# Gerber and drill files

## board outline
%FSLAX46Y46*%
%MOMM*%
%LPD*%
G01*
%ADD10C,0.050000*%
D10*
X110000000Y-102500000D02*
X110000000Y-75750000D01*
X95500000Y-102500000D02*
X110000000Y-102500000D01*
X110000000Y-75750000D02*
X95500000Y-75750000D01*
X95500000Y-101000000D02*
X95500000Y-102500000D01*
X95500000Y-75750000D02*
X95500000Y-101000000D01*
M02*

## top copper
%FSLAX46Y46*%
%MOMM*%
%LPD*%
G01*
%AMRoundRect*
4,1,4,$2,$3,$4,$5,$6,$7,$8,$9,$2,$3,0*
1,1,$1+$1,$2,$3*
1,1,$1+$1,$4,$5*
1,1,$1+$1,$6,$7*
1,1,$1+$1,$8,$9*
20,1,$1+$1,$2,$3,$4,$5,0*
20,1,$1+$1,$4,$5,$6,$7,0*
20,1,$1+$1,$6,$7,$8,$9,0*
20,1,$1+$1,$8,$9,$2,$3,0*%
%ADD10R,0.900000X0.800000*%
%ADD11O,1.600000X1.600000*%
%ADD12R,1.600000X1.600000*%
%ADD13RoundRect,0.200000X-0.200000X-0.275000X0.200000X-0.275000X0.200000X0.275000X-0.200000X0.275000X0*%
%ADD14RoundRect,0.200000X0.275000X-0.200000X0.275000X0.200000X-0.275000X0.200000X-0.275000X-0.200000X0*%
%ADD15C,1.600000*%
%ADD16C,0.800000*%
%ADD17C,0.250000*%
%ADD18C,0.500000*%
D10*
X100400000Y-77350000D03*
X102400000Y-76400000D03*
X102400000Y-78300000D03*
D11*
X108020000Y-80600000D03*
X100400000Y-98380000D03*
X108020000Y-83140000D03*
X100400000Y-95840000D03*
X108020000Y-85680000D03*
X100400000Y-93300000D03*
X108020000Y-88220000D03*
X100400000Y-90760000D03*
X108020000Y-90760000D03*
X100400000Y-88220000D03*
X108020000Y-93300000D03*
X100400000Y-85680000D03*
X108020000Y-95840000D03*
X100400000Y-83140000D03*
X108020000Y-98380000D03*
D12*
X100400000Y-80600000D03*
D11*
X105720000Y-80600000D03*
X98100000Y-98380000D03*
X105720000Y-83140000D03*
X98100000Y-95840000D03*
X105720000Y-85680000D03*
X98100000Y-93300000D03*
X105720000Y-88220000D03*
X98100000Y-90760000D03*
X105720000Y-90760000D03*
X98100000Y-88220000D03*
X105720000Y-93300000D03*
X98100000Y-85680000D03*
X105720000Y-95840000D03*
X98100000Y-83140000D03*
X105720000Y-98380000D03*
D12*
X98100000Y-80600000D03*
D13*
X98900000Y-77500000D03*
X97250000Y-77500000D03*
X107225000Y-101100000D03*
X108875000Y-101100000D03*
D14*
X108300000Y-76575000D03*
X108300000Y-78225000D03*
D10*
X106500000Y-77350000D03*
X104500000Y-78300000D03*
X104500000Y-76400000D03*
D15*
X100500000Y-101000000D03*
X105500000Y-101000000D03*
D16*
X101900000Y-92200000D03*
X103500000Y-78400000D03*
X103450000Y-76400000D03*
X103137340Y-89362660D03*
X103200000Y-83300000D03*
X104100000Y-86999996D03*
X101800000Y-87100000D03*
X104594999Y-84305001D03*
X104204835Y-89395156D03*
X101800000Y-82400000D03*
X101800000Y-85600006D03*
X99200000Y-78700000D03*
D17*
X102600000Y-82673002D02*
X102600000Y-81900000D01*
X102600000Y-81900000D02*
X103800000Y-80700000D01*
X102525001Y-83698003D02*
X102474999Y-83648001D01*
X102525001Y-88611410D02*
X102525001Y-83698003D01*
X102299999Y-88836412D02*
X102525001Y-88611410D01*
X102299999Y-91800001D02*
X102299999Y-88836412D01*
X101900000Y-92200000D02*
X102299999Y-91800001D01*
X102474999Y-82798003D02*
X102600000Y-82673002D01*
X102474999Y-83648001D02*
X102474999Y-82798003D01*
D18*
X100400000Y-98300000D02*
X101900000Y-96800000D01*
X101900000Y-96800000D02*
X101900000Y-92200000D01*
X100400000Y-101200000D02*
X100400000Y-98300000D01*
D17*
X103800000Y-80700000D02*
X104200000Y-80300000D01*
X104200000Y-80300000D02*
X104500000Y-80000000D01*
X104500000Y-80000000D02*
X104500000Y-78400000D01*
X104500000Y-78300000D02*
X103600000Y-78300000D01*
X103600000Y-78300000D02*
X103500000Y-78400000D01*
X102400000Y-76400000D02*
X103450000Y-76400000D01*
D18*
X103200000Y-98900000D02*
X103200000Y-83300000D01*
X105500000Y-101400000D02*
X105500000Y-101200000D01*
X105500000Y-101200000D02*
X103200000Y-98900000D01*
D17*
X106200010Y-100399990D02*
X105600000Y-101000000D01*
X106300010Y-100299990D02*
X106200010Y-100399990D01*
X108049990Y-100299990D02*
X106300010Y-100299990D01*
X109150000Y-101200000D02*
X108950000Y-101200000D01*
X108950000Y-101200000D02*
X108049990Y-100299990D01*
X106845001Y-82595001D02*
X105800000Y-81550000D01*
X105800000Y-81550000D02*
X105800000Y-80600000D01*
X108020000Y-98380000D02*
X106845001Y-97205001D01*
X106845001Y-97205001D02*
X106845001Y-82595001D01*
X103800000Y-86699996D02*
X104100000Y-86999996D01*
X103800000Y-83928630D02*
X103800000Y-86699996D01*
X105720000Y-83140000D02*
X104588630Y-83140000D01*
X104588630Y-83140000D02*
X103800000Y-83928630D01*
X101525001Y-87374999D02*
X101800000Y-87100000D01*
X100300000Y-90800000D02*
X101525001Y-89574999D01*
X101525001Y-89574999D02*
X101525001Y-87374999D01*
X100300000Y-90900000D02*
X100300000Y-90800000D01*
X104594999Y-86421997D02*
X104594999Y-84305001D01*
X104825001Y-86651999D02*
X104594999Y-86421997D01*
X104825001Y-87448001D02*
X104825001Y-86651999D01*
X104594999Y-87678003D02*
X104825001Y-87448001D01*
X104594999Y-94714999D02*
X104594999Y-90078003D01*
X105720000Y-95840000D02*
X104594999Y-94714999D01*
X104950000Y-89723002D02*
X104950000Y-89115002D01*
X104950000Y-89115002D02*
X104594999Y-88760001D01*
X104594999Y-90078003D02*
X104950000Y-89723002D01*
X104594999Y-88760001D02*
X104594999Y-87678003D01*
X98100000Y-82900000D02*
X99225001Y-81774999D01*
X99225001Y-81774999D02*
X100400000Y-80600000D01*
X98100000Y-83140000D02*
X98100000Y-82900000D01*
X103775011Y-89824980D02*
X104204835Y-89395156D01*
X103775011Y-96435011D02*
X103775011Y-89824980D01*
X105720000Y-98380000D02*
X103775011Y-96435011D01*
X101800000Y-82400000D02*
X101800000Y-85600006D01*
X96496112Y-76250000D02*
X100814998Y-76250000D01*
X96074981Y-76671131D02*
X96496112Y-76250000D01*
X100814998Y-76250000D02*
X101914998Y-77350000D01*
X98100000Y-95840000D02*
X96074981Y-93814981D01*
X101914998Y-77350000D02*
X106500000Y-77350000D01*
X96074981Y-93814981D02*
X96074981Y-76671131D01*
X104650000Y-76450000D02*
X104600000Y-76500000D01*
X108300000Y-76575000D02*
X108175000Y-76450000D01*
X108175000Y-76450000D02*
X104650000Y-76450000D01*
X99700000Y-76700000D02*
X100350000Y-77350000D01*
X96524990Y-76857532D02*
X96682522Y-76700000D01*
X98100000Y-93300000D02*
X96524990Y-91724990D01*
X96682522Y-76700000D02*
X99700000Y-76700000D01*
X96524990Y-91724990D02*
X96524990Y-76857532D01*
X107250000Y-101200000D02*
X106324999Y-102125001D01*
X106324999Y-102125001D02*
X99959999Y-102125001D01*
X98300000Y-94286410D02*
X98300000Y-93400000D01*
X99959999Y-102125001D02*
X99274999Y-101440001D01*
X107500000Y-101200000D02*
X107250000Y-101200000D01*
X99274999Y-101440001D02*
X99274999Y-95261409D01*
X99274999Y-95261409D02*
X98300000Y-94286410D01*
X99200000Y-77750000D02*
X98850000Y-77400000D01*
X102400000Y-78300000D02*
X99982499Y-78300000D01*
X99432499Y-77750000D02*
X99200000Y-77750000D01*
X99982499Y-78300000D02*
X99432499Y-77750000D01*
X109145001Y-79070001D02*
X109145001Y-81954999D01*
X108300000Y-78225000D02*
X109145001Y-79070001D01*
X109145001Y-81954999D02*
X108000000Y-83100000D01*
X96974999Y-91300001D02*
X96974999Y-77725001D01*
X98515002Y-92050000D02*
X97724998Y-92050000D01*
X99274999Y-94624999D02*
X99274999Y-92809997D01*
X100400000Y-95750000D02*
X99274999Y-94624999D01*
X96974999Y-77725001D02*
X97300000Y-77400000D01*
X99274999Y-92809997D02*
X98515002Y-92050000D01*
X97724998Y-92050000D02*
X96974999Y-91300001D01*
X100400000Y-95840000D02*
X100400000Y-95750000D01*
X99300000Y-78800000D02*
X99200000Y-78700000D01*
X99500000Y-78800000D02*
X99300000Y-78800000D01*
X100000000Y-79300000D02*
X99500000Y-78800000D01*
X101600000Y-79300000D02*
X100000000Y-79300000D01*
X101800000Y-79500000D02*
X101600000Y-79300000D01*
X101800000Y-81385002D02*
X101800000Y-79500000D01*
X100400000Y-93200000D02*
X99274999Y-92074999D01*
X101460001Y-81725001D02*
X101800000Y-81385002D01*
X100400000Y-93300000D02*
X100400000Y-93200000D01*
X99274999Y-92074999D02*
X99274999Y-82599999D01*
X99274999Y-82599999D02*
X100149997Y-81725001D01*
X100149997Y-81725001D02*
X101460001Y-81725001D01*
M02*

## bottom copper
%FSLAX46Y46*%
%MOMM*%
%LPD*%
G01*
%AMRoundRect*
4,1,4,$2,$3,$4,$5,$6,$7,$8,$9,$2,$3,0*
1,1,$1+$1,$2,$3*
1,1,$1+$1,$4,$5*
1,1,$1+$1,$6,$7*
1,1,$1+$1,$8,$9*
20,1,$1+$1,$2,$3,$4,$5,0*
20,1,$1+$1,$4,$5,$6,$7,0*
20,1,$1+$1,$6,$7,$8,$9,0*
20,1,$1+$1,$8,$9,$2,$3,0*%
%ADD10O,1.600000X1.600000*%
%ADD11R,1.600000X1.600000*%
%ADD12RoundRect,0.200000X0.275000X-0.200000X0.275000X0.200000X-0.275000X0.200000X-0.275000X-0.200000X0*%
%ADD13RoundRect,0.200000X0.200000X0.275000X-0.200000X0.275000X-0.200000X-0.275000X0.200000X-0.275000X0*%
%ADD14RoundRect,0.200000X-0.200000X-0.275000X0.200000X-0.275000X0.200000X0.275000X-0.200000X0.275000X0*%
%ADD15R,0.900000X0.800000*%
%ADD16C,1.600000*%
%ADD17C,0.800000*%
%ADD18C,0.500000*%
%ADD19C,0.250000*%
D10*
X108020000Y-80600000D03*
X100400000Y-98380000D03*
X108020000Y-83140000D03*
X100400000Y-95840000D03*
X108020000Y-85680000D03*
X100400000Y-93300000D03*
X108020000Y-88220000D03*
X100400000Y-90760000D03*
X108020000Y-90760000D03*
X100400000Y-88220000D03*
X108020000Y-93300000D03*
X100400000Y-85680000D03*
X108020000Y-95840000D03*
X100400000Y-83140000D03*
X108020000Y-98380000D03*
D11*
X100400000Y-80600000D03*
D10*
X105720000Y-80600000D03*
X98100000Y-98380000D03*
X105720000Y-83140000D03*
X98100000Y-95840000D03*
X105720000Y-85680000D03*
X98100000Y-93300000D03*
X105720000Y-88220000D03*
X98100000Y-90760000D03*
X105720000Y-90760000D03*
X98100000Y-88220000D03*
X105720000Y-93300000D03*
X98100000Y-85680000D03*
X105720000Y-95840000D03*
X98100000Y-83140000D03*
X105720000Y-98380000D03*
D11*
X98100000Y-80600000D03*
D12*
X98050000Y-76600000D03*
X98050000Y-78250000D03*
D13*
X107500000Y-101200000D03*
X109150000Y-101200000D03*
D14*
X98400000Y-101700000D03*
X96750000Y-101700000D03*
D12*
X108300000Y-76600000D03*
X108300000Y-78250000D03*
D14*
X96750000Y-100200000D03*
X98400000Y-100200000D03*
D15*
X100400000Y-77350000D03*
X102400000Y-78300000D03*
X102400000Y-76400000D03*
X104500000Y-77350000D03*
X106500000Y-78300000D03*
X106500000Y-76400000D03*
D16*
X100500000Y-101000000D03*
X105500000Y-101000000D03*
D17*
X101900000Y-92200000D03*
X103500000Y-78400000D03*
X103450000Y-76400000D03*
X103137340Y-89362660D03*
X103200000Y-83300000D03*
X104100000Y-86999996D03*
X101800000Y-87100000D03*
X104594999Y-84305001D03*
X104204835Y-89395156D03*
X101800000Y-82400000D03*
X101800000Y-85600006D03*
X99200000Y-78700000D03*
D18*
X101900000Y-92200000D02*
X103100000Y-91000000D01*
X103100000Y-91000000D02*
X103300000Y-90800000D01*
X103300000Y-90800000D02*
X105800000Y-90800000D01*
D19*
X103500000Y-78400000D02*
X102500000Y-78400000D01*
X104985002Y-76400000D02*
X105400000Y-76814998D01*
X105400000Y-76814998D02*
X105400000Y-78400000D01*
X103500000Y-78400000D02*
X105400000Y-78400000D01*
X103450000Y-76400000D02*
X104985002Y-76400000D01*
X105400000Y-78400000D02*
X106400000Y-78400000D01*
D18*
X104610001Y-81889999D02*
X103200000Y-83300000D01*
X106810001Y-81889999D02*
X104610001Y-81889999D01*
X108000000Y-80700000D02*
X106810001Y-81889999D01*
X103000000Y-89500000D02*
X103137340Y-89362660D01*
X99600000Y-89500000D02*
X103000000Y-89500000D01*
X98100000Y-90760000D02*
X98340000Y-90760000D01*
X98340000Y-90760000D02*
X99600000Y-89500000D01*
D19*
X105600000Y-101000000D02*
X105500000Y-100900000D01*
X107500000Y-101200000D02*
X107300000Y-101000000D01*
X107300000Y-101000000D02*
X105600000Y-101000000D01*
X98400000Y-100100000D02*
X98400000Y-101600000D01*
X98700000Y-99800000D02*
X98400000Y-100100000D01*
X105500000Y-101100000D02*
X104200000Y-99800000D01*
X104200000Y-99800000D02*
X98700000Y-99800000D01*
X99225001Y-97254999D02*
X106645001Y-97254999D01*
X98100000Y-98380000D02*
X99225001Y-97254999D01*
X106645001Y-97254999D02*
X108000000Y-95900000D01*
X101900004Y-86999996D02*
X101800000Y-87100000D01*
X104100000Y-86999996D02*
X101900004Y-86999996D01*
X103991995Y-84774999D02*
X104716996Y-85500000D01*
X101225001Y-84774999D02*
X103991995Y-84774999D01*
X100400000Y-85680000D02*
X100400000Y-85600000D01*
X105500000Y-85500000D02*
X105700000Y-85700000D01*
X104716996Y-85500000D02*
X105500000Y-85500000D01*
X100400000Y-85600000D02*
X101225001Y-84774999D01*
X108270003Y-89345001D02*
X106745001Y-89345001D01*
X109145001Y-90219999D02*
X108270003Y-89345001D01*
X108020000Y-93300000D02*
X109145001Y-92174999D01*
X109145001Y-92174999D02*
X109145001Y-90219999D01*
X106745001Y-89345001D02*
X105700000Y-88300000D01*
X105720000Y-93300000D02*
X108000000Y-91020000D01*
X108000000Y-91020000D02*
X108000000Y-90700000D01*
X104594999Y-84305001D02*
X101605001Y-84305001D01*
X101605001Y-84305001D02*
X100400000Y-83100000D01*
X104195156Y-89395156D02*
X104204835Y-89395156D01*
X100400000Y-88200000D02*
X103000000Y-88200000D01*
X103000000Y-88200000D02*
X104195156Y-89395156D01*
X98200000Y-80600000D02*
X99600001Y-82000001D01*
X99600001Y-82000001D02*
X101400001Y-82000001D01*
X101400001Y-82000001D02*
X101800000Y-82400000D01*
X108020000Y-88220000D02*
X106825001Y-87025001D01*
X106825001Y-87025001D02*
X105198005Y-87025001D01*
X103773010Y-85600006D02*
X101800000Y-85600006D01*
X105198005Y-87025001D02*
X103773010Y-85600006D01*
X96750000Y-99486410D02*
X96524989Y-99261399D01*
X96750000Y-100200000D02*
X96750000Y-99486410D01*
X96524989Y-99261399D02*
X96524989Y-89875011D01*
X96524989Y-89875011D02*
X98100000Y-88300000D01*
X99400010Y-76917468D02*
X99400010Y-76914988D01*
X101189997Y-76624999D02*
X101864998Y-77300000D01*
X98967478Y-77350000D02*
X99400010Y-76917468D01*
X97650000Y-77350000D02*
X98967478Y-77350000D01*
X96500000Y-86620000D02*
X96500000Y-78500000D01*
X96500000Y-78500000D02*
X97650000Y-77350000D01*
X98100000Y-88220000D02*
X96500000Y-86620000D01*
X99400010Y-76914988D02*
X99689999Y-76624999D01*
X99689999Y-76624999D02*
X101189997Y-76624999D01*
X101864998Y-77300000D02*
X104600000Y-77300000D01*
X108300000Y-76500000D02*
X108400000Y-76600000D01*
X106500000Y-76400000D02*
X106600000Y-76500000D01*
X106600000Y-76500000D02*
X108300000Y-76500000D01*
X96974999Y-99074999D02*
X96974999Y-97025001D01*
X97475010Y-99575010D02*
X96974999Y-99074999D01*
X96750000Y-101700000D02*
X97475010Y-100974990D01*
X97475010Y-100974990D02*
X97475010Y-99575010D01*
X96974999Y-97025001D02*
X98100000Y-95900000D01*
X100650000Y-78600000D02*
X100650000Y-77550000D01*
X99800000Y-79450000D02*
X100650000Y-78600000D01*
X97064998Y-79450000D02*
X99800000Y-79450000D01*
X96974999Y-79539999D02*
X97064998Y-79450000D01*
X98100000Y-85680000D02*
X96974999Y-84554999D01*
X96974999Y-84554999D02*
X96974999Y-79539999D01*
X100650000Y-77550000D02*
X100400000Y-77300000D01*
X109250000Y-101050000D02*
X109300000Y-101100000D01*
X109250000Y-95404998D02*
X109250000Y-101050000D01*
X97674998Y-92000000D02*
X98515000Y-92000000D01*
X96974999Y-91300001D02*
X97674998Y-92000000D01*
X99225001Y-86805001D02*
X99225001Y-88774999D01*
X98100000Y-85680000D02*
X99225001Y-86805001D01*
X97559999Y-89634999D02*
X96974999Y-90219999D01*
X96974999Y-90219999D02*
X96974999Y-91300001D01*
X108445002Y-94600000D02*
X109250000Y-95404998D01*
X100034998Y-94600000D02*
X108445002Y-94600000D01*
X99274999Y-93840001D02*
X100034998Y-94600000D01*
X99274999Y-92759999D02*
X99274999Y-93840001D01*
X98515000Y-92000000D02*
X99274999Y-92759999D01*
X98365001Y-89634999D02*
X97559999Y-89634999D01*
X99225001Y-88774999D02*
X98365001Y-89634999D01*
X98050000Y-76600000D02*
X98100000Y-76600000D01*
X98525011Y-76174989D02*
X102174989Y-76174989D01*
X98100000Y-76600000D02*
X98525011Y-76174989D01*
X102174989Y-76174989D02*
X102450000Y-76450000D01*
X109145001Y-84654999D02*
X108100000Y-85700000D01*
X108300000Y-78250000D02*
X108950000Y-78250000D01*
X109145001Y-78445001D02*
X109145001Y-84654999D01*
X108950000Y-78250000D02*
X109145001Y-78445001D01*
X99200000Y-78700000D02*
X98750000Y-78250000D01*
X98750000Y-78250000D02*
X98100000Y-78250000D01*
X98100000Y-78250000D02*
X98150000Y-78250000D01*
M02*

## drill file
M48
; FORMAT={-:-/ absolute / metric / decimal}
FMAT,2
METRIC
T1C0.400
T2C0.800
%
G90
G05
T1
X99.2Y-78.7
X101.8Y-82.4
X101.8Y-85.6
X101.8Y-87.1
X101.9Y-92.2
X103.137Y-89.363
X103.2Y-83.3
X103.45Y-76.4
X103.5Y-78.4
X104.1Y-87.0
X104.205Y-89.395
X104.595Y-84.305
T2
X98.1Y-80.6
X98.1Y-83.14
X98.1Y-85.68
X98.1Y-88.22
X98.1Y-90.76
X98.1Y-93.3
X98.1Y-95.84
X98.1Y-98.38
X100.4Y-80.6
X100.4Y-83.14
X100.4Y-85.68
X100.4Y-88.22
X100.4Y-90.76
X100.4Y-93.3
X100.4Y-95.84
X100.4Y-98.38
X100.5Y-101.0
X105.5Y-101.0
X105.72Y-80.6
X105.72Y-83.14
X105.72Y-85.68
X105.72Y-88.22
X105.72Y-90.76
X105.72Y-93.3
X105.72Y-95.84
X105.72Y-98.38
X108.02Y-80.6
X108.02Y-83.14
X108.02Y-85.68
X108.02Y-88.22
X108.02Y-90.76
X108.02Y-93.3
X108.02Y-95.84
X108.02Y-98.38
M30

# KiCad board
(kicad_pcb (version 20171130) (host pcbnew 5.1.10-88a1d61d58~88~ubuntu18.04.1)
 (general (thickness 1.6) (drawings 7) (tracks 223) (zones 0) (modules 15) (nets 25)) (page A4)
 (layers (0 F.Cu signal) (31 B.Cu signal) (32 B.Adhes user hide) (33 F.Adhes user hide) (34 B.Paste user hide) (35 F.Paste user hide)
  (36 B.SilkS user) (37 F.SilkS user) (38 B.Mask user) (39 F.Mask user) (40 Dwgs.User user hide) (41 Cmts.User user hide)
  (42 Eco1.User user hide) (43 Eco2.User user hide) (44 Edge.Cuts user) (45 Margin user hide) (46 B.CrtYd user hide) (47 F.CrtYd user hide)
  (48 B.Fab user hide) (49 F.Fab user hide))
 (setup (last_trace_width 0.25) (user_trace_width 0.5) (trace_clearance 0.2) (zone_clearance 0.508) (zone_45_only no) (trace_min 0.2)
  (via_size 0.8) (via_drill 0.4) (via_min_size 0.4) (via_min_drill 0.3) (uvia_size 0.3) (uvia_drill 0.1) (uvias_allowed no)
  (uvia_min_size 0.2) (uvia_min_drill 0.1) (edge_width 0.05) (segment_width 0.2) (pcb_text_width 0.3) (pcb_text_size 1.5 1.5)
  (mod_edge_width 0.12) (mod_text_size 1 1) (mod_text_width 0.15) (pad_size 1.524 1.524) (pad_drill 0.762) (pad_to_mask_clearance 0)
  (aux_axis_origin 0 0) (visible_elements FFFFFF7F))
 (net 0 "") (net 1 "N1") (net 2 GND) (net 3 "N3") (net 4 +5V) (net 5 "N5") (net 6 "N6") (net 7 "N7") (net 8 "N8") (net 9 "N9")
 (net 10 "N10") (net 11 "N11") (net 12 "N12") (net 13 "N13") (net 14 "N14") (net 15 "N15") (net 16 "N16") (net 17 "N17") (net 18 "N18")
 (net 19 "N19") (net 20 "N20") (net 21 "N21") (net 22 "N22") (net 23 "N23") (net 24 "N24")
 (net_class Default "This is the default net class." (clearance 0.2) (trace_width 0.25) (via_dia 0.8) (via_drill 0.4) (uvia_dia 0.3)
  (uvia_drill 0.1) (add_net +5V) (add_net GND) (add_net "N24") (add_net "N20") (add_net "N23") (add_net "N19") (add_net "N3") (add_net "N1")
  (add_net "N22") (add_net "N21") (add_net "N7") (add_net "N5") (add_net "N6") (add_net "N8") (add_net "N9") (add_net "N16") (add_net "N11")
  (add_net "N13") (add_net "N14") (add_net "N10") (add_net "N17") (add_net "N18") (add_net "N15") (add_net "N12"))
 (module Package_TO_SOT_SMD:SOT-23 (layer F.Cu) (at 101.4 77.35 180)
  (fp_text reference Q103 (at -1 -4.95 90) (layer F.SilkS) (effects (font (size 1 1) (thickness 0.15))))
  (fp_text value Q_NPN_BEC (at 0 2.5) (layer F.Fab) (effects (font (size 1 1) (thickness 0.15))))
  (pad 3 smd rect (at 1 0 180) (size 0.9 0.8) (layers F.Cu F.Paste F.Mask) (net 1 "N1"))
  (pad 2 smd rect (at -1 0.95 180) (size 0.9 0.8) (layers F.Cu F.Paste F.Mask) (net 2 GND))
  (pad 1 smd rect (at -1 -0.95 180) (size 0.9 0.8) (layers F.Cu F.Paste F.Mask) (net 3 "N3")))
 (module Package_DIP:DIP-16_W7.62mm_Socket (layer F.Cu) (at 100.4 80.6)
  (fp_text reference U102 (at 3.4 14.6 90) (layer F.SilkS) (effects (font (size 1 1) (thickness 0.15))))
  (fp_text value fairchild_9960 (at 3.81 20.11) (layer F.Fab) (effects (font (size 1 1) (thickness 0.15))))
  (pad 16 thru_hole oval (at 7.62 0) (size 1.6 1.6) (drill 0.8) (layers *.Cu *.Mask) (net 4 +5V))
  (pad 8 thru_hole oval (at 0 17.78) (size 1.6 1.6) (drill 0.8) (layers *.Cu *.Mask) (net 2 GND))
  (pad 15 thru_hole oval (at 7.62 2.54) (size 1.6 1.6) (drill 0.8) (layers *.Cu *.Mask) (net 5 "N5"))
  (pad 7 thru_hole oval (at 0 15.24) (size 1.6 1.6) (drill 0.8) (layers *.Cu *.Mask) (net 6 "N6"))
  (pad 14 thru_hole oval (at 7.62 5.08) (size 1.6 1.6) (drill 0.8) (layers *.Cu *.Mask) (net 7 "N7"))
  (pad 6 thru_hole oval (at 0 12.7) (size 1.6 1.6) (drill 0.8) (layers *.Cu *.Mask) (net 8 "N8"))
  (pad 13 thru_hole oval (at 7.62 7.62) (size 1.6 1.6) (drill 0.8) (layers *.Cu *.Mask) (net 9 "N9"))
  (pad 5 thru_hole oval (at 0 10.16) (size 1.6 1.6) (drill 0.8) (layers *.Cu *.Mask) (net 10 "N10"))
  (pad 12 thru_hole oval (at 7.62 10.16) (size 1.6 1.6) (drill 0.8) (layers *.Cu *.Mask) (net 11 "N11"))
  (pad 4 thru_hole oval (at 0 7.62) (size 1.6 1.6) (drill 0.8) (layers *.Cu *.Mask) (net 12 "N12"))
  (pad 11 thru_hole oval (at 7.62 12.7) (size 1.6 1.6) (drill 0.8) (layers *.Cu *.Mask) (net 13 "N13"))
  (pad 3 thru_hole oval (at 0 5.08) (size 1.6 1.6) (drill 0.8) (layers *.Cu *.Mask) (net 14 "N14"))
  (pad 10 thru_hole oval (at 7.62 15.24) (size 1.6 1.6) (drill 0.8) (layers *.Cu *.Mask) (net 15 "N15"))
  (pad 2 thru_hole oval (at 0 2.54) (size 1.6 1.6) (drill 0.8) (layers *.Cu *.Mask) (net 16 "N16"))
  (pad 9 thru_hole oval (at 7.62 17.78) (size 1.6 1.6) (drill 0.8) (layers *.Cu *.Mask) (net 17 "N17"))
  (pad 1 thru_hole rect (at 0 0) (size 1.6 1.6) (drill 0.8) (layers *.Cu *.Mask) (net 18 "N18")))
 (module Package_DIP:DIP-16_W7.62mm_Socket (layer F.Cu) (at 98.1 80.6)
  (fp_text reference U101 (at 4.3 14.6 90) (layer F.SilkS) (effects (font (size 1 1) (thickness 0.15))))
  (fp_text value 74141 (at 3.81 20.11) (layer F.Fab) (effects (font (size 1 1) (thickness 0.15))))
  (pad 16 thru_hole oval (at 7.62 0) (size 1.6 1.6) (drill 0.8) (layers *.Cu *.Mask) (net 17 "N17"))
  (pad 8 thru_hole oval (at 0 17.78) (size 1.6 1.6) (drill 0.8) (layers *.Cu *.Mask) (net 15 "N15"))
  (pad 15 thru_hole oval (at 7.62 2.54) (size 1.6 1.6) (drill 0.8) (layers *.Cu *.Mask) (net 10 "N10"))
  (pad 7 thru_hole oval (at 0 15.24) (size 1.6 1.6) (drill 0.8) (layers *.Cu *.Mask) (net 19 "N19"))
  (pad 14 thru_hole oval (at 7.62 5.08) (size 1.6 1.6) (drill 0.8) (layers *.Cu *.Mask) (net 14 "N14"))
  (pad 6 thru_hole oval (at 0 12.7) (size 1.6 1.6) (drill 0.8) (layers *.Cu *.Mask) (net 1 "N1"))
  (pad 13 thru_hole oval (at 7.62 7.62) (size 1.6 1.6) (drill 0.8) (layers *.Cu *.Mask) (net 13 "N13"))
  (pad 5 thru_hole oval (at 0 10.16) (size 1.6 1.6) (drill 0.8) (layers *.Cu *.Mask) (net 4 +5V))
  (pad 12 thru_hole oval (at 7.62 10.16) (size 1.6 1.6) (drill 0.8) (layers *.Cu *.Mask) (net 2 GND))
  (pad 4 thru_hole oval (at 0 7.62) (size 1.6 1.6) (drill 0.8) (layers *.Cu *.Mask) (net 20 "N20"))
  (pad 11 thru_hole oval (at 7.62 12.7) (size 1.6 1.6) (drill 0.8) (layers *.Cu *.Mask) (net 11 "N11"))
  (pad 3 thru_hole oval (at 0 5.08) (size 1.6 1.6) (drill 0.8) (layers *.Cu *.Mask) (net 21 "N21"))
  (pad 10 thru_hole oval (at 7.62 15.24) (size 1.6 1.6) (drill 0.8) (layers *.Cu *.Mask) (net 16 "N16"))
  (pad 2 thru_hole oval (at 0 2.54) (size 1.6 1.6) (drill 0.8) (layers *.Cu *.Mask) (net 18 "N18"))
  (pad 9 thru_hole oval (at 7.62 17.78) (size 1.6 1.6) (drill 0.8) (layers *.Cu *.Mask) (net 12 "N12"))
  (pad 1 thru_hole rect (at 0 0) (size 1.6 1.6) (drill 0.8) (layers *.Cu *.Mask) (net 9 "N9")))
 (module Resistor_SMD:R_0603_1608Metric (layer B.Cu) (at 98.05 77.425 90)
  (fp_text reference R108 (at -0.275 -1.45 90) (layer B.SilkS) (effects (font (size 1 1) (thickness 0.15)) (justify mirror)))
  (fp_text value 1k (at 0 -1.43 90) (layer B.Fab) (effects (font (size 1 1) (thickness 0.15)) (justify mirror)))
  (pad 2 smd roundrect (at 0.825 0 90) (size 0.8 0.95) (layers B.Cu B.Paste B.Mask) (roundrect_rratio 0.25) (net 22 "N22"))
  (pad 1 smd roundrect (at -0.825 0 90) (size 0.8 0.95) (layers B.Cu B.Paste B.Mask) (roundrect_rratio 0.25) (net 8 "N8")))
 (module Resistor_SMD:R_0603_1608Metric (layer B.Cu) (at 108.325 101.2 180)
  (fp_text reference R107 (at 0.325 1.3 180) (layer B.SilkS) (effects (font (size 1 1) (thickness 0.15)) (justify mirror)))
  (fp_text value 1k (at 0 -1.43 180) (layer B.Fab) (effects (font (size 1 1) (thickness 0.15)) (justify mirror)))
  (pad 2 smd roundrect (at 0.825 0 180) (size 0.8 0.95) (layers B.Cu B.Paste B.Mask) (roundrect_rratio 0.25) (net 4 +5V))
  (pad 1 smd roundrect (at -0.825 0 180) (size 0.8 0.95) (layers B.Cu B.Paste B.Mask) (roundrect_rratio 0.25) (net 21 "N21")))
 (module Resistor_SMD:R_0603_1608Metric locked (layer F.Cu) (at 98.075 77.5)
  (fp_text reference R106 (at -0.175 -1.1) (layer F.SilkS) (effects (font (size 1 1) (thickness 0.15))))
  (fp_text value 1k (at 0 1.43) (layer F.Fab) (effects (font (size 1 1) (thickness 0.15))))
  (pad 2 smd roundrect (at 0.825 0) (size 0.8 0.95) (layers F.Cu F.Paste F.Mask) (roundrect_rratio 0.25) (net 3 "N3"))
  (pad 1 smd roundrect (at -0.825 0) (size 0.8 0.95) (layers F.Cu F.Paste F.Mask) (roundrect_rratio 0.25) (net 6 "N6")))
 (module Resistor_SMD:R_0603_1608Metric (layer F.Cu) (at 108.05 101.1)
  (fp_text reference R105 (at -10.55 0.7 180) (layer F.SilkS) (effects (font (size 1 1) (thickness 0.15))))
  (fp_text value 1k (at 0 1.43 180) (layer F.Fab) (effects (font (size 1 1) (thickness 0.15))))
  (pad 1 smd roundrect (at -0.825 0) (size 0.8 0.95) (layers F.Cu F.Paste F.Mask) (roundrect_rratio 0.25) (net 1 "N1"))
  (pad 2 smd roundrect (at 0.825 0) (size 0.8 0.95) (layers F.Cu F.Paste F.Mask) (roundrect_rratio 0.25) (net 4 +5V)))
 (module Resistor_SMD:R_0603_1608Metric (layer F.Cu) (at 108.3 77.4 90)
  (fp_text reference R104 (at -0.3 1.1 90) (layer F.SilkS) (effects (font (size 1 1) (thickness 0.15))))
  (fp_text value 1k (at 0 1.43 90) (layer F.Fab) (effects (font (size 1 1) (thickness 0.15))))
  (pad 2 smd roundrect (at 0.825 0 90) (size 0.8 0.95) (layers F.Cu F.Paste F.Mask) (roundrect_rratio 0.25) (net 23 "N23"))
  (pad 1 smd roundrect (at -0.825 0 90) (size 0.8 0.95) (layers F.Cu F.Paste F.Mask) (roundrect_rratio 0.25) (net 5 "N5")))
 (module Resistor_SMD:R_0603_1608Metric (layer B.Cu) (at 97.575 101.7)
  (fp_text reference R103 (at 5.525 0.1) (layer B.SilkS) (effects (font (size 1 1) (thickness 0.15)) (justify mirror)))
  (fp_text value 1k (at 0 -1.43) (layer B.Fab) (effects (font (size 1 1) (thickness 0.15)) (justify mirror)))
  (pad 2 smd roundrect (at 0.825 0) (size 0.8 0.95) (layers B.Cu B.Paste B.Mask) (roundrect_rratio 0.25) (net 4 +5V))
  (pad 1 smd roundrect (at -0.825 0) (size 0.8 0.95) (layers B.Cu B.Paste B.Mask) (roundrect_rratio 0.25) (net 19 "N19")))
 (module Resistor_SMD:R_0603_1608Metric (layer B.Cu) (at 108.3 77.425 90)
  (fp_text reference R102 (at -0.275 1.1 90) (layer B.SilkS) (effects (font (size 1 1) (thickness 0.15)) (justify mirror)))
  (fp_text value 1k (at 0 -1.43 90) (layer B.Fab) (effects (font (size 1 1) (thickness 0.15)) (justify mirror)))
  (pad 2 smd roundrect (at 0.825 0 90) (size 0.8 0.95) (layers B.Cu B.Paste B.Mask) (roundrect_rratio 0.25) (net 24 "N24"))
  (pad 1 smd roundrect (at -0.825 0 90) (size 0.8 0.95) (layers B.Cu B.Paste B.Mask) (roundrect_rratio 0.25) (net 7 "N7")))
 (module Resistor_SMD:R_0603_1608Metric (layer B.Cu) (at 97.575 100.2)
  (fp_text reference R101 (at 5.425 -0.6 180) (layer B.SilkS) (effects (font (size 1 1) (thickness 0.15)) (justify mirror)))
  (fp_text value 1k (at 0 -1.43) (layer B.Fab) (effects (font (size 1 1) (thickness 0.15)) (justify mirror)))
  (pad 1 smd roundrect (at -0.825 0) (size 0.8 0.95) (layers B.Cu B.Paste B.Mask) (roundrect_rratio 0.25) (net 20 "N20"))
  (pad 2 smd roundrect (at 0.825 0) (size 0.8 0.95) (layers B.Cu B.Paste B.Mask) (roundrect_rratio 0.25) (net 4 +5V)))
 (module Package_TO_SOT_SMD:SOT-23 (layer B.Cu) (at 101.4 77.35 180)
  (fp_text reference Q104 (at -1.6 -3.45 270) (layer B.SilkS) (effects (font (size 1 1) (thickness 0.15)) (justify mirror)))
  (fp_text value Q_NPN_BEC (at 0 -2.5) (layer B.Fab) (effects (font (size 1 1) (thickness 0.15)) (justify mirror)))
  (pad 3 smd rect (at 1 0 180) (size 0.9 0.8) (layers B.Cu B.Paste B.Mask) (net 21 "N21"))
  (pad 2 smd rect (at -1 -0.95 180) (size 0.9 0.8) (layers B.Cu B.Paste B.Mask) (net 2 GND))
  (pad 1 smd rect (at -1 0.95 180) (size 0.9 0.8) (layers B.Cu B.Paste B.Mask) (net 22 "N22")))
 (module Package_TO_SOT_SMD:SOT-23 (layer F.Cu) (at 105.5 77.35)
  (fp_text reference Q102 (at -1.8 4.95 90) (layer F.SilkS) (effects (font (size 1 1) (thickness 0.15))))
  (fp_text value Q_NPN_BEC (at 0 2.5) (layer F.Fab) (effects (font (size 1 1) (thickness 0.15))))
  (pad 3 smd rect (at 1 0) (size 0.9 0.8) (layers F.Cu F.Paste F.Mask) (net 19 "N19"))
  (pad 2 smd rect (at -1 0.95) (size 0.9 0.8) (layers F.Cu F.Paste F.Mask) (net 2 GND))
  (pad 1 smd rect (at -1 -0.95) (size 0.9 0.8) (layers F.Cu F.Paste F.Mask) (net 23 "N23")))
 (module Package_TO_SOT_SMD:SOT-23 (layer B.Cu) (at 105.5 77.35 180)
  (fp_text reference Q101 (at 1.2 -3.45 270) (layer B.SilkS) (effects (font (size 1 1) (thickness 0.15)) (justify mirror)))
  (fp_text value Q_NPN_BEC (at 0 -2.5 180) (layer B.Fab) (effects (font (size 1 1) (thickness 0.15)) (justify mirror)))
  (pad 3 smd rect (at 1 0 180) (size 0.9 0.8) (layers B.Cu B.Paste B.Mask) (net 20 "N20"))
  (pad 2 smd rect (at -1 -0.95 180) (size 0.9 0.8) (layers B.Cu B.Paste B.Mask) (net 2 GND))
  (pad 1 smd rect (at -1 0.95 180) (size 0.9 0.8) (layers B.Cu B.Paste B.Mask) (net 24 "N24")))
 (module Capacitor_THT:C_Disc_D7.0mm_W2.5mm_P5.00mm (layer F.Cu) (at 105.5 101 180)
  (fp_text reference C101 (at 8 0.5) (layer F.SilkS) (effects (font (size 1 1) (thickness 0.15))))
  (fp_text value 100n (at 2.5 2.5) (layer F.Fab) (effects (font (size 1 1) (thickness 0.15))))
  (pad 2 thru_hole circle (at 5 0 180) (size 1.6 1.6) (drill 0.8) (layers *.Cu *.Mask) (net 2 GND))
  (pad 1 thru_hole circle (at 0 0 180) (size 1.6 1.6) (drill 0.8) (layers *.Cu *.Mask) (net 4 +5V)))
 (gr_line (start 110 102.5) (end 110 75.75) (layer Edge.Cuts) (width 0.05))
 (gr_line (start 95.5 102.5) (end 110 102.5) (layer Edge.Cuts) (width 0.05))
 (gr_line (start 110 75.75) (end 95.5 75.75) (layer Edge.Cuts) (width 0.05))
 (gr_line (start 95.5 101) (end 95.5 102.5) (layer Edge.Cuts) (width 0.05))
 (gr_line (start 95.5 75.75) (end 95.5 101) (layer Edge.Cuts) (width 0.05))
 (via (at 101.9 92.2) (size 0.8) (drill 0.4) (layers F.Cu B.Cu) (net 2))
 (segment (start 101.9 92.2) (end 103.1 91) (width 0.5) (layer B.Cu) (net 2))
 (segment (start 103.1 91) (end 103.3 90.8) (width 0.5) (layer B.Cu) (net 2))
 (segment (start 103.3 90.8) (end 105.8 90.8) (width 0.5) (layer B.Cu) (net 2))
 (segment (start 102.6 82.673002) (end 102.6 81.9) (width 0.25) (layer F.Cu) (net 2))
 (segment (start 102.6 81.9) (end 103.8 80.7) (width 0.25) (layer F.Cu) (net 2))
 (segment (start 102.525001 83.698003) (end 102.474999 83.648001) (width 0.25) (layer F.Cu) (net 2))
 (segment (start 102.525001 88.61141) (end 102.525001 83.698003) (width 0.25) (layer F.Cu) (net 2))
 (segment (start 102.299999 88.836412) (end 102.525001 88.61141) (width 0.25) (layer F.Cu) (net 2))
 (segment (start 102.299999 91.800001) (end 102.299999 88.836412) (width 0.25) (layer F.Cu) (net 2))
 (segment (start 101.9 92.2) (end 102.299999 91.800001) (width 0.25) (layer F.Cu) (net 2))
 (segment (start 102.474999 82.798003) (end 102.6 82.673002) (width 0.25) (layer F.Cu) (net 2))
 (segment (start 102.474999 83.648001) (end 102.474999 82.798003) (width 0.25) (layer F.Cu) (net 2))
 (segment (start 100.4 98.3) (end 101.9 96.8) (width 0.5) (layer F.Cu) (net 2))
 (segment (start 101.9 96.8) (end 101.9 92.2) (width 0.5) (layer F.Cu) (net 2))
 (segment (start 100.4 101.2) (end 100.4 98.3) (width 0.5) (layer F.Cu) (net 2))
 (segment (start 103.8 80.7) (end 104.2 80.3) (width 0.25) (layer F.Cu) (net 2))
 (segment (start 104.2 80.3) (end 104.5 80) (width 0.25) (layer F.Cu) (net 2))
 (segment (start 104.5 80) (end 104.5 78.4) (width 0.25) (layer F.Cu) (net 2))
 (segment (start 104.5 78.3) (end 103.6 78.3) (width 0.25) (layer F.Cu) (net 2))
 (via (at 103.5 78.4) (size 0.8) (drill 0.4) (layers F.Cu B.Cu) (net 2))
 (segment (start 103.6 78.3) (end 103.5 78.4) (width 0.25) (layer F.Cu) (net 2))
 (segment (start 103.5 78.4) (end 102.5 78.4) (width 0.25) (layer B.Cu) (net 2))
 (via (at 103.45 76.4) (size 0.8) (drill 0.4) (layers F.Cu B.Cu) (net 2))
 (segment (start 102.4 76.4) (end 103.45 76.4) (width 0.25) (layer F.Cu) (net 2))
 (segment (start 104.985002 76.4) (end 105.4 76.814998) (width 0.25) (layer B.Cu) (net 2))
 (segment (start 105.4 76.814998) (end 105.4 78.4) (width 0.25) (layer B.Cu) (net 2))
 (segment (start 103.5 78.4) (end 105.4 78.4) (width 0.25) (layer B.Cu) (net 2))
 (segment (start 103.45 76.4) (end 104.985002 76.4) (width 0.25) (layer B.Cu) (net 2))
 (segment (start 105.4 78.4) (end 106.4 78.4) (width 0.25) (layer B.Cu) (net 2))
 (via (at 103.13734 89.36266) (size 0.8) (drill 0.4) (layers F.Cu B.Cu) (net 4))
 (segment (start 104.610001 81.889999) (end 103.2 83.3) (width 0.5) (layer B.Cu) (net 4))
 (segment (start 106.810001 81.889999) (end 104.610001 81.889999) (width 0.5) (layer B.Cu) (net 4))
 (via (at 103.2 83.3) (size 0.8) (drill 0.4) (layers F.Cu B.Cu) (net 4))
 (segment (start 108 80.7) (end 106.810001 81.889999) (width 0.5) (layer B.Cu) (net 4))
 (segment (start 103.2 98.9) (end 103.2 83.3) (width 0.5) (layer F.Cu) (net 4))
 (segment (start 105.5 101.4) (end 105.5 101.2) (width 0.5) (layer F.Cu) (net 4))
 (segment (start 105.5 101.2) (end 103.2 98.9) (width 0.5) (layer F.Cu) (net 4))
 (segment (start 103 89.5) (end 103.13734 89.36266) (width 0.5) (layer B.Cu) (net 4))
 (segment (start 99.6 89.5) (end 103 89.5) (width 0.5) (layer B.Cu) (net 4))
 (segment (start 98.1 90.76) (end 98.34 90.76) (width 0.5) (layer B.Cu) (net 4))
 (segment (start 98.34 90.76) (end 99.6 89.5) (width 0.5) (layer B.Cu) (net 4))
 (segment (start 105.6 101) (end 105.5 100.9) (width 0.25) (layer B.Cu) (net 4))
 (segment (start 107.5 101.2) (end 107.3 101) (width 0.25) (layer B.Cu) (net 4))
 (segment (start 107.3 101) (end 105.6 101) (width 0.25) (layer B.Cu) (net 4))
 (segment (start 98.4 100.1) (end 98.4 101.6) (width 0.25) (layer B.Cu) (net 4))
 (segment (start 98.7 99.8) (end 98.4 100.1) (width 0.25) (layer B.Cu) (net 4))
 (segment (start 105.5 101.1) (end 104.2 99.8) (width 0.25) (layer B.Cu) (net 4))
 (segment (start 104.2 99.8) (end 98.7 99.8) (width 0.25) (layer B.Cu) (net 4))
 (segment (start 106.20001 100.39999) (end 105.6 101) (width 0.25) (layer F.Cu) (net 4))
 (segment (start 106.30001 100.29999) (end 106.20001 100.39999) (width 0.25) (layer F.Cu) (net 4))
 (segment (start 108.04999 100.29999) (end 106.30001 100.29999) (width 0.25) (layer F.Cu) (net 4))
 (segment (start 109.15 101.2) (end 108.95 101.2) (width 0.25) (layer F.Cu) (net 4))
 (segment (start 108.95 101.2) (end 108.04999 100.29999) (width 0.25) (layer F.Cu) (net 4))
 (segment (start 106.845001 82.595001) (end 105.8 81.55) (width 0.25) (layer F.Cu) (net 17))
 (segment (start 105.8 81.55) (end 105.8 80.6) (width 0.25) (layer F.Cu) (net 17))
 (segment (start 108.02 98.38) (end 106.845001 97.205001) (width 0.25) (layer F.Cu) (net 17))
 (segment (start 106.845001 97.205001) (end 106.845001 82.595001) (width 0.25) (layer F.Cu) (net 17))
 (segment (start 99.225001 97.254999) (end 106.645001 97.254999) (width 0.25) (layer B.Cu) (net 15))
 (segment (start 98.1 98.38) (end 99.225001 97.254999) (width 0.25) (layer B.Cu) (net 15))
 (segment (start 106.645001 97.254999) (end 108 95.9) (width 0.25) (layer B.Cu) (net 15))
 (via (at 104.1 86.999996) (size 0.8) (drill 0.4) (layers F.Cu B.Cu) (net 10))
 (segment (start 103.8 86.699996) (end 104.1 86.999996) (width 0.25) (layer F.Cu) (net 10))
 (segment (start 103.8 83.92863) (end 103.8 86.699996) (width 0.25) (layer F.Cu) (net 10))
 (segment (start 105.72 83.14) (end 104.58863 83.14) (width 0.25) (layer F.Cu) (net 10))
 (segment (start 104.58863 83.14) (end 103.8 83.92863) (width 0.25) (layer F.Cu) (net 10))
 (segment (start 101.900004 86.999996) (end 101.8 87.1) (width 0.25) (layer B.Cu) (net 10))
 (segment (start 104.1 86.999996) (end 101.900004 86.999996) (width 0.25) (layer B.Cu) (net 10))
 (via (at 101.8 87.1) (size 0.8) (drill 0.4) (layers F.Cu B.Cu) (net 10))
 (segment (start 101.525001 87.374999) (end 101.8 87.1) (width 0.25) (layer F.Cu) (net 10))
 (segment (start 100.3 90.8) (end 101.525001 89.574999) (width 0.25) (layer F.Cu) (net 10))
 (segment (start 101.525001 89.574999) (end 101.525001 87.374999) (width 0.25) (layer F.Cu) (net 10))
 (segment (start 100.3 90.9) (end 100.3 90.8) (width 0.25) (layer F.Cu) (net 10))
 (segment (start 103.991995 84.774999) (end 104.716996 85.5) (width 0.25) (layer B.Cu) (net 14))
 (segment (start 101.225001 84.774999) (end 103.991995 84.774999) (width 0.25) (layer B.Cu) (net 14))
 (segment (start 100.4 85.68) (end 100.4 85.6) (width 0.25) (layer B.Cu) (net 14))
 (segment (start 105.5 85.5) (end 105.7 85.7) (width 0.25) (layer B.Cu) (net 14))
 (segment (start 104.716996 85.5) (end 105.5 85.5) (width 0.25) (layer B.Cu) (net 14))
 (segment (start 100.4 85.6) (end 101.225001 84.774999) (width 0.25) (layer B.Cu) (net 14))
 (segment (start 108.270003 89.345001) (end 106.745001 89.345001) (width 0.25) (layer B.Cu) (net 13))
 (segment (start 109.145001 90.219999) (end 108.270003 89.345001) (width 0.25) (layer B.Cu) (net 13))
 (segment (start 108.02 93.3) (end 109.145001 92.174999) (width 0.25) (layer B.Cu) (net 13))
 (segment (start 109.145001 92.174999) (end 109.145001 90.219999) (width 0.25) (layer B.Cu) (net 13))
 (segment (start 106.745001 89.345001) (end 105.7 88.3) (width 0.25) (layer B.Cu) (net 13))
 (segment (start 105.72 93.3) (end 108 91.02) (width 0.25) (layer B.Cu) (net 11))
 (segment (start 108 91.02) (end 108 90.7) (width 0.25) (layer B.Cu) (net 11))
 (via (at 104.594999 84.305001) (size 0.8) (drill 0.4) (layers F.Cu B.Cu) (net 16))
 (segment (start 104.594999 84.305001) (end 101.605001 84.305001) (width 0.25) (layer B.Cu) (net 16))
 (segment (start 101.605001 84.305001) (end 100.4 83.1) (width 0.25) (layer B.Cu) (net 16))
 (segment (start 104.594999 86.421997) (end 104.594999 84.305001) (width 0.25) (layer F.Cu) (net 16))
 (segment (start 104.825001 86.651999) (end 104.594999 86.421997) (width 0.25) (layer F.Cu) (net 16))
 (segment (start 104.825001 87.448001) (end 104.825001 86.651999) (width 0.25) (layer F.Cu) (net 16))
 (segment (start 104.594999 87.678003) (end 104.825001 87.448001) (width 0.25) (layer F.Cu) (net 16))
 (segment (start 104.594999 94.714999) (end 104.594999 90.078003) (width 0.25) (layer F.Cu) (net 16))
 (segment (start 105.72 95.84) (end 104.594999 94.714999) (width 0.25) (layer F.Cu) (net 16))
 (segment (start 104.95 89.723002) (end 104.95 89.115002) (width 0.25) (layer F.Cu) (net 16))
 (segment (start 104.95 89.115002) (end 104.594999 88.760001) (width 0.25) (layer F.Cu) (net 16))
 (segment (start 104.594999 90.078003) (end 104.95 89.723002) (width 0.25) (layer F.Cu) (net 16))
 (segment (start 104.594999 88.760001) (end 104.594999 87.678003) (width 0.25) (layer F.Cu) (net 16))
 (segment (start 98.1 82.9) (end 99.225001 81.774999) (width 0.25) (layer F.Cu) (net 18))
 (segment (start 99.225001 81.774999) (end 100.4 80.6) (width 0.25) (layer F.Cu) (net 18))
 (segment (start 98.1 83.14) (end 98.1 82.9) (width 0.25) (layer F.Cu) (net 18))
 (via (at 104.204835 89.395156) (size 0.8) (drill 0.4) (layers F.Cu B.Cu) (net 12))
 (segment (start 103.775011 89.82498) (end 104.204835 89.395156) (width 0.25) (layer F.Cu) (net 12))
 (segment (start 103.775011 96.435011) (end 103.775011 89.82498) (width 0.25) (layer F.Cu) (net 12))
 (segment (start 105.72 98.38) (end 103.775011 96.435011) (width 0.25) (layer F.Cu) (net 12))
 (segment (start 104.195156 89.395156) (end 104.204835 89.395156) (width 0.25) (layer B.Cu) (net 12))
 (segment (start 100.4 88.2) (end 103 88.2) (width 0.25) (layer B.Cu) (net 12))
 (segment (start 103 88.2) (end 104.195156 89.395156) (width 0.25) (layer B.Cu) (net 12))
 (segment (start 98.2 80.6) (end 99.600001 82.000001) (width 0.25) (layer B.Cu) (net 9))
 (segment (start 99.600001 82.000001) (end 101.400001 82.000001) (width 0.25) (layer B.Cu) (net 9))
 (segment (start 101.400001 82.000001) (end 101.8 82.4) (width 0.25) (layer B.Cu) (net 9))
 (via (at 101.8 82.4) (size 0.8) (drill 0.4) (layers F.Cu B.Cu) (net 9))
 (segment (start 101.8 82.4) (end 101.8 85.600006) (width 0.25) (layer F.Cu) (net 9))
 (segment (start 108.02 88.22) (end 106.825001 87.025001) (width 0.25) (layer B.Cu) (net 9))
 (via (at 101.8 85.600006) (size 0.8) (drill 0.4) (layers F.Cu B.Cu) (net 9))
 (segment (start 106.825001 87.025001) (end 105.198005 87.025001) (width 0.25) (layer B.Cu) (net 9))
 (segment (start 103.77301 85.600006) (end 101.8 85.600006) (width 0.25) (layer B.Cu) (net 9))
 (segment (start 105.198005 87.025001) (end 103.77301 85.600006) (width 0.25) (layer B.Cu) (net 9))
 (segment (start 96.75 99.48641) (end 96.524989 99.261399) (width 0.25) (layer B.Cu) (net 20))
 (segment (start 96.75 100.2) (end 96.75 99.48641) (width 0.25) (layer B.Cu) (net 20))
 (segment (start 96.524989 99.261399) (end 96.524989 89.875011) (width 0.25) (layer B.Cu) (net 20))
 (segment (start 96.524989 89.875011) (end 98.1 88.3) (width 0.25) (layer B.Cu) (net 20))
 (segment (start 99.40001 76.917468) (end 99.40001 76.914988) (width 0.25) (layer B.Cu) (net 20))
 (segment (start 101.189997 76.624999) (end 101.864998 77.3) (width 0.25) (layer B.Cu) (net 20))
 (segment (start 98.967478 77.35) (end 99.40001 76.917468) (width 0.25) (layer B.Cu) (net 20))
 (segment (start 97.65 77.35) (end 98.967478 77.35) (width 0.25) (layer B.Cu) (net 20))
 (segment (start 96.5 86.62) (end 96.5 78.5) (width 0.25) (layer B.Cu) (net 20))
 (segment (start 96.5 78.5) (end 97.65 77.35) (width 0.25) (layer B.Cu) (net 20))
 (segment (start 98.1 88.22) (end 96.5 86.62) (width 0.25) (layer B.Cu) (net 20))
 (segment (start 99.40001 76.914988) (end 99.689999 76.624999) (width 0.25) (layer B.Cu) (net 20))
 (segment (start 99.689999 76.624999) (end 101.189997 76.624999) (width 0.25) (layer B.Cu) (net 20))
 (segment (start 101.864998 77.3) (end 104.6 77.3) (width 0.25) (layer B.Cu) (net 20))
 (segment (start 108.3 76.5) (end 108.4 76.6) (width 0.25) (layer B.Cu) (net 24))
 (segment (start 106.5 76.4) (end 106.6 76.5) (width 0.25) (layer B.Cu) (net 24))
 (segment (start 106.6 76.5) (end 108.3 76.5) (width 0.25) (layer B.Cu) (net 24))
 (segment (start 96.974999 99.074999) (end 96.974999 97.025001) (width 0.25) (layer B.Cu) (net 19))
 (segment (start 97.47501 99.57501) (end 96.974999 99.074999) (width 0.25) (layer B.Cu) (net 19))
 (segment (start 96.75 101.7) (end 97.47501 100.97499) (width 0.25) (layer B.Cu) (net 19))
 (segment (start 97.47501 100.97499) (end 97.47501 99.57501) (width 0.25) (layer B.Cu) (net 19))
 (segment (start 96.974999 97.025001) (end 98.1 95.9) (width 0.25) (layer B.Cu) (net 19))
 (segment (start 96.496112 76.25) (end 100.814998 76.25) (width 0.25) (layer F.Cu) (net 19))
 (segment (start 96.074981 76.671131) (end 96.496112 76.25) (width 0.25) (layer F.Cu) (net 19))
 (segment (start 100.814998 76.25) (end 101.914998 77.35) (width 0.25) (layer F.Cu) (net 19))
 (segment (start 98.1 95.84) (end 96.074981 93.814981) (width 0.25) (layer F.Cu) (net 19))
 (segment (start 101.914998 77.35) (end 106.5 77.35) (width 0.25) (layer F.Cu) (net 19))
 (segment (start 96.074981 93.814981) (end 96.074981 76.671131) (width 0.25) (layer F.Cu) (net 19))
 (segment (start 104.65 76.45) (end 104.6 76.5) (width 0.25) (layer F.Cu) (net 23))
 (segment (start 108.3 76.575) (end 108.175 76.45) (width 0.25) (layer F.Cu) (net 23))
 (segment (start 108.175 76.45) (end 104.65 76.45) (width 0.25) (layer F.Cu) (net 23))
 (segment (start 99.7 76.7) (end 100.35 77.35) (width 0.25) (layer F.Cu) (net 1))
 (segment (start 96.52499 76.857532) (end 96.682522 76.7) (width 0.25) (layer F.Cu) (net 1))
 (segment (start 98.1 93.3) (end 96.52499 91.72499) (width 0.25) (layer F.Cu) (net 1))
 (segment (start 96.682522 76.7) (end 99.7 76.7) (width 0.25) (layer F.Cu) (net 1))
 (segment (start 96.52499 91.72499) (end 96.52499 76.857532) (width 0.25) (layer F.Cu) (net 1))
 (segment (start 107.25 101.2) (end 106.324999 102.125001) (width 0.25) (layer F.Cu) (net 1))
 (segment (start 106.324999 102.125001) (end 99.959999 102.125001) (width 0.25) (layer F.Cu) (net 1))
 (segment (start 98.3 94.28641) (end 98.3 93.4) (width 0.25) (layer F.Cu) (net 1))
 (segment (start 99.959999 102.125001) (end 99.274999 101.440001) (width 0.25) (layer F.Cu) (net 1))
 (segment (start 107.5 101.2) (end 107.25 101.2) (width 0.25) (layer F.Cu) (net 1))
 (segment (start 99.274999 101.440001) (end 99.274999 95.261409) (width 0.25) (layer F.Cu) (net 1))
 (segment (start 99.274999 95.261409) (end 98.3 94.28641) (width 0.25) (layer F.Cu) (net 1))
 (segment (start 99.2 77.75) (end 98.85 77.4) (width 0.25) (layer F.Cu) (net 3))
 (segment (start 102.4 78.3) (end 99.982499 78.3) (width 0.25) (layer F.Cu) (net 3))
 (segment (start 99.432499 77.75) (end 99.2 77.75) (width 0.25) (layer F.Cu) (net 3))
 (segment (start 99.982499 78.3) (end 99.432499 77.75) (width 0.25) (layer F.Cu) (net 3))
 (segment (start 100.65 78.6) (end 100.65 77.55) (width 0.25) (layer B.Cu) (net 21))
 (segment (start 99.8 79.45) (end 100.65 78.6) (width 0.25) (layer B.Cu) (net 21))
 (segment (start 97.064998 79.45) (end 99.8 79.45) (width 0.25) (layer B.Cu) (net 21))
 (segment (start 96.974999 79.539999) (end 97.064998 79.45) (width 0.25) (layer B.Cu) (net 21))
 (segment (start 98.1 85.68) (end 96.974999 84.554999) (width 0.25) (layer B.Cu) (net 21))
 (segment (start 96.974999 84.554999) (end 96.974999 79.539999) (width 0.25) (layer B.Cu) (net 21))
 (segment (start 100.65 77.55) (end 100.4 77.3) (width 0.25) (layer B.Cu) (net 21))
 (segment (start 109.25 101.05) (end 109.3 101.1) (width 0.25) (layer B.Cu) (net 21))
 (segment (start 109.25 95.404998) (end 109.25 101.05) (width 0.25) (layer B.Cu) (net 21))
 (segment (start 97.674998 92) (end 98.515 92) (width 0.25) (layer B.Cu) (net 21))
 (segment (start 96.974999 91.300001) (end 97.674998 92) (width 0.25) (layer B.Cu) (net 21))
 (segment (start 99.225001 86.805001) (end 99.225001 88.774999) (width 0.25) (layer B.Cu) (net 21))
 (segment (start 98.1 85.68) (end 99.225001 86.805001) (width 0.25) (layer B.Cu) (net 21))
 (segment (start 97.559999 89.634999) (end 96.974999 90.219999) (width 0.25) (layer B.Cu) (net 21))
 (segment (start 96.974999 90.219999) (end 96.974999 91.300001) (width 0.25) (layer B.Cu) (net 21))
 (segment (start 108.445002 94.6) (end 109.25 95.404998) (width 0.25) (layer B.Cu) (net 21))
 (segment (start 100.034998 94.6) (end 108.445002 94.6) (width 0.25) (layer B.Cu) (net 21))
 (segment (start 99.274999 93.840001) (end 100.034998 94.6) (width 0.25) (layer B.Cu) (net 21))
 (segment (start 99.274999 92.759999) (end 99.274999 93.840001) (width 0.25) (layer B.Cu) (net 21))
 (segment (start 98.515 92) (end 99.274999 92.759999) (width 0.25) (layer B.Cu) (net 21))
 (segment (start 98.365001 89.634999) (end 97.559999 89.634999) (width 0.25) (layer B.Cu) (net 21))
 (segment (start 99.225001 88.774999) (end 98.365001 89.634999) (width 0.25) (layer B.Cu) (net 21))
 (segment (start 98.05 76.6) (end 98.1 76.6) (width 0.25) (layer B.Cu) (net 22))
 (segment (start 98.525011 76.174989) (end 102.174989 76.174989) (width 0.25) (layer B.Cu) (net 22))
 (segment (start 98.1 76.6) (end 98.525011 76.174989) (width 0.25) (layer B.Cu) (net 22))
 (segment (start 102.174989 76.174989) (end 102.45 76.45) (width 0.25) (layer B.Cu) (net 22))
 (segment (start 109.145001 84.654999) (end 108.1 85.7) (width 0.25) (layer B.Cu) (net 7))
 (segment (start 108.3 78.25) (end 108.95 78.25) (width 0.25) (layer B.Cu) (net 7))
 (segment (start 109.145001 78.445001) (end 109.145001 84.654999) (width 0.25) (layer B.Cu) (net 7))
 (segment (start 108.95 78.25) (end 109.145001 78.445001) (width 0.25) (layer B.Cu) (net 7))
 (segment (start 109.145001 79.070001) (end 109.145001 81.954999) (width 0.25) (layer F.Cu) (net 5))
 (segment (start 108.3 78.225) (end 109.145001 79.070001) (width 0.25) (layer F.Cu) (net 5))
 (segment (start 109.145001 81.954999) (end 108 83.1) (width 0.25) (layer F.Cu) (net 5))
 (segment (start 96.974999 91.300001) (end 96.974999 77.725001) (width 0.25) (layer F.Cu) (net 6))
 (segment (start 98.515002 92.05) (end 97.724998 92.05) (width 0.25) (layer F.Cu) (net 6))
 (segment (start 99.274999 94.624999) (end 99.274999 92.809997) (width 0.25) (layer F.Cu) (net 6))
 (segment (start 100.4 95.75) (end 99.274999 94.624999) (width 0.25) (layer F.Cu) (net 6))
 (segment (start 96.974999 77.725001) (end 97.3 77.4) (width 0.25) (layer F.Cu) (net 6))
 (segment (start 99.274999 92.809997) (end 98.515002 92.05) (width 0.25) (layer F.Cu) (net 6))
 (segment (start 97.724998 92.05) (end 96.974999 91.300001) (width 0.25) (layer F.Cu) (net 6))
 (segment (start 100.4 95.84) (end 100.4 95.75) (width 0.25) (layer F.Cu) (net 6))
 (via (at 99.2 78.7) (size 0.8) (drill 0.4) (layers F.Cu B.Cu) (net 8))
 (segment (start 99.2 78.7) (end 98.75 78.25) (width 0.25) (layer B.Cu) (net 8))
 (segment (start 98.75 78.25) (end 98.1 78.25) (width 0.25) (layer B.Cu) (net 8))
 (segment (start 98.1 78.25) (end 98.15 78.25) (width 0.25) (layer B.Cu) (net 8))
 (segment (start 99.3 78.8) (end 99.2 78.7) (width 0.25) (layer F.Cu) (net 8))
 (segment (start 99.5 78.8) (end 99.3 78.8) (width 0.25) (layer F.Cu) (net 8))
 (segment (start 100 79.3) (end 99.5 78.8) (width 0.25) (layer F.Cu) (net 8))
 (segment (start 101.6 79.3) (end 100 79.3) (width 0.25) (layer F.Cu) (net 8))
 (segment (start 101.8 79.5) (end 101.6 79.3) (width 0.25) (layer F.Cu) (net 8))
 (segment (start 101.8 81.385002) (end 101.8 79.5) (width 0.25) (layer F.Cu) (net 8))
 (segment (start 100.4 93.2) (end 99.274999 92.074999) (width 0.25) (layer F.Cu) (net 8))
 (segment (start 101.460001 81.725001) (end 101.8 81.385002) (width 0.25) (layer F.Cu) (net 8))
 (segment (start 100.4 93.3) (end 100.4 93.2) (width 0.25) (layer F.Cu) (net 8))
 (segment (start 99.274999 92.074999) (end 99.274999 82.599999) (width 0.25) (layer F.Cu) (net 8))
 (segment (start 99.274999 82.599999) (end 100.149997 81.725001) (width 0.25) (layer F.Cu) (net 8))
 (segment (start 100.149997 81.725001) (end 101.460001 81.725001) (width 0.25) (layer F.Cu) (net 8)))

